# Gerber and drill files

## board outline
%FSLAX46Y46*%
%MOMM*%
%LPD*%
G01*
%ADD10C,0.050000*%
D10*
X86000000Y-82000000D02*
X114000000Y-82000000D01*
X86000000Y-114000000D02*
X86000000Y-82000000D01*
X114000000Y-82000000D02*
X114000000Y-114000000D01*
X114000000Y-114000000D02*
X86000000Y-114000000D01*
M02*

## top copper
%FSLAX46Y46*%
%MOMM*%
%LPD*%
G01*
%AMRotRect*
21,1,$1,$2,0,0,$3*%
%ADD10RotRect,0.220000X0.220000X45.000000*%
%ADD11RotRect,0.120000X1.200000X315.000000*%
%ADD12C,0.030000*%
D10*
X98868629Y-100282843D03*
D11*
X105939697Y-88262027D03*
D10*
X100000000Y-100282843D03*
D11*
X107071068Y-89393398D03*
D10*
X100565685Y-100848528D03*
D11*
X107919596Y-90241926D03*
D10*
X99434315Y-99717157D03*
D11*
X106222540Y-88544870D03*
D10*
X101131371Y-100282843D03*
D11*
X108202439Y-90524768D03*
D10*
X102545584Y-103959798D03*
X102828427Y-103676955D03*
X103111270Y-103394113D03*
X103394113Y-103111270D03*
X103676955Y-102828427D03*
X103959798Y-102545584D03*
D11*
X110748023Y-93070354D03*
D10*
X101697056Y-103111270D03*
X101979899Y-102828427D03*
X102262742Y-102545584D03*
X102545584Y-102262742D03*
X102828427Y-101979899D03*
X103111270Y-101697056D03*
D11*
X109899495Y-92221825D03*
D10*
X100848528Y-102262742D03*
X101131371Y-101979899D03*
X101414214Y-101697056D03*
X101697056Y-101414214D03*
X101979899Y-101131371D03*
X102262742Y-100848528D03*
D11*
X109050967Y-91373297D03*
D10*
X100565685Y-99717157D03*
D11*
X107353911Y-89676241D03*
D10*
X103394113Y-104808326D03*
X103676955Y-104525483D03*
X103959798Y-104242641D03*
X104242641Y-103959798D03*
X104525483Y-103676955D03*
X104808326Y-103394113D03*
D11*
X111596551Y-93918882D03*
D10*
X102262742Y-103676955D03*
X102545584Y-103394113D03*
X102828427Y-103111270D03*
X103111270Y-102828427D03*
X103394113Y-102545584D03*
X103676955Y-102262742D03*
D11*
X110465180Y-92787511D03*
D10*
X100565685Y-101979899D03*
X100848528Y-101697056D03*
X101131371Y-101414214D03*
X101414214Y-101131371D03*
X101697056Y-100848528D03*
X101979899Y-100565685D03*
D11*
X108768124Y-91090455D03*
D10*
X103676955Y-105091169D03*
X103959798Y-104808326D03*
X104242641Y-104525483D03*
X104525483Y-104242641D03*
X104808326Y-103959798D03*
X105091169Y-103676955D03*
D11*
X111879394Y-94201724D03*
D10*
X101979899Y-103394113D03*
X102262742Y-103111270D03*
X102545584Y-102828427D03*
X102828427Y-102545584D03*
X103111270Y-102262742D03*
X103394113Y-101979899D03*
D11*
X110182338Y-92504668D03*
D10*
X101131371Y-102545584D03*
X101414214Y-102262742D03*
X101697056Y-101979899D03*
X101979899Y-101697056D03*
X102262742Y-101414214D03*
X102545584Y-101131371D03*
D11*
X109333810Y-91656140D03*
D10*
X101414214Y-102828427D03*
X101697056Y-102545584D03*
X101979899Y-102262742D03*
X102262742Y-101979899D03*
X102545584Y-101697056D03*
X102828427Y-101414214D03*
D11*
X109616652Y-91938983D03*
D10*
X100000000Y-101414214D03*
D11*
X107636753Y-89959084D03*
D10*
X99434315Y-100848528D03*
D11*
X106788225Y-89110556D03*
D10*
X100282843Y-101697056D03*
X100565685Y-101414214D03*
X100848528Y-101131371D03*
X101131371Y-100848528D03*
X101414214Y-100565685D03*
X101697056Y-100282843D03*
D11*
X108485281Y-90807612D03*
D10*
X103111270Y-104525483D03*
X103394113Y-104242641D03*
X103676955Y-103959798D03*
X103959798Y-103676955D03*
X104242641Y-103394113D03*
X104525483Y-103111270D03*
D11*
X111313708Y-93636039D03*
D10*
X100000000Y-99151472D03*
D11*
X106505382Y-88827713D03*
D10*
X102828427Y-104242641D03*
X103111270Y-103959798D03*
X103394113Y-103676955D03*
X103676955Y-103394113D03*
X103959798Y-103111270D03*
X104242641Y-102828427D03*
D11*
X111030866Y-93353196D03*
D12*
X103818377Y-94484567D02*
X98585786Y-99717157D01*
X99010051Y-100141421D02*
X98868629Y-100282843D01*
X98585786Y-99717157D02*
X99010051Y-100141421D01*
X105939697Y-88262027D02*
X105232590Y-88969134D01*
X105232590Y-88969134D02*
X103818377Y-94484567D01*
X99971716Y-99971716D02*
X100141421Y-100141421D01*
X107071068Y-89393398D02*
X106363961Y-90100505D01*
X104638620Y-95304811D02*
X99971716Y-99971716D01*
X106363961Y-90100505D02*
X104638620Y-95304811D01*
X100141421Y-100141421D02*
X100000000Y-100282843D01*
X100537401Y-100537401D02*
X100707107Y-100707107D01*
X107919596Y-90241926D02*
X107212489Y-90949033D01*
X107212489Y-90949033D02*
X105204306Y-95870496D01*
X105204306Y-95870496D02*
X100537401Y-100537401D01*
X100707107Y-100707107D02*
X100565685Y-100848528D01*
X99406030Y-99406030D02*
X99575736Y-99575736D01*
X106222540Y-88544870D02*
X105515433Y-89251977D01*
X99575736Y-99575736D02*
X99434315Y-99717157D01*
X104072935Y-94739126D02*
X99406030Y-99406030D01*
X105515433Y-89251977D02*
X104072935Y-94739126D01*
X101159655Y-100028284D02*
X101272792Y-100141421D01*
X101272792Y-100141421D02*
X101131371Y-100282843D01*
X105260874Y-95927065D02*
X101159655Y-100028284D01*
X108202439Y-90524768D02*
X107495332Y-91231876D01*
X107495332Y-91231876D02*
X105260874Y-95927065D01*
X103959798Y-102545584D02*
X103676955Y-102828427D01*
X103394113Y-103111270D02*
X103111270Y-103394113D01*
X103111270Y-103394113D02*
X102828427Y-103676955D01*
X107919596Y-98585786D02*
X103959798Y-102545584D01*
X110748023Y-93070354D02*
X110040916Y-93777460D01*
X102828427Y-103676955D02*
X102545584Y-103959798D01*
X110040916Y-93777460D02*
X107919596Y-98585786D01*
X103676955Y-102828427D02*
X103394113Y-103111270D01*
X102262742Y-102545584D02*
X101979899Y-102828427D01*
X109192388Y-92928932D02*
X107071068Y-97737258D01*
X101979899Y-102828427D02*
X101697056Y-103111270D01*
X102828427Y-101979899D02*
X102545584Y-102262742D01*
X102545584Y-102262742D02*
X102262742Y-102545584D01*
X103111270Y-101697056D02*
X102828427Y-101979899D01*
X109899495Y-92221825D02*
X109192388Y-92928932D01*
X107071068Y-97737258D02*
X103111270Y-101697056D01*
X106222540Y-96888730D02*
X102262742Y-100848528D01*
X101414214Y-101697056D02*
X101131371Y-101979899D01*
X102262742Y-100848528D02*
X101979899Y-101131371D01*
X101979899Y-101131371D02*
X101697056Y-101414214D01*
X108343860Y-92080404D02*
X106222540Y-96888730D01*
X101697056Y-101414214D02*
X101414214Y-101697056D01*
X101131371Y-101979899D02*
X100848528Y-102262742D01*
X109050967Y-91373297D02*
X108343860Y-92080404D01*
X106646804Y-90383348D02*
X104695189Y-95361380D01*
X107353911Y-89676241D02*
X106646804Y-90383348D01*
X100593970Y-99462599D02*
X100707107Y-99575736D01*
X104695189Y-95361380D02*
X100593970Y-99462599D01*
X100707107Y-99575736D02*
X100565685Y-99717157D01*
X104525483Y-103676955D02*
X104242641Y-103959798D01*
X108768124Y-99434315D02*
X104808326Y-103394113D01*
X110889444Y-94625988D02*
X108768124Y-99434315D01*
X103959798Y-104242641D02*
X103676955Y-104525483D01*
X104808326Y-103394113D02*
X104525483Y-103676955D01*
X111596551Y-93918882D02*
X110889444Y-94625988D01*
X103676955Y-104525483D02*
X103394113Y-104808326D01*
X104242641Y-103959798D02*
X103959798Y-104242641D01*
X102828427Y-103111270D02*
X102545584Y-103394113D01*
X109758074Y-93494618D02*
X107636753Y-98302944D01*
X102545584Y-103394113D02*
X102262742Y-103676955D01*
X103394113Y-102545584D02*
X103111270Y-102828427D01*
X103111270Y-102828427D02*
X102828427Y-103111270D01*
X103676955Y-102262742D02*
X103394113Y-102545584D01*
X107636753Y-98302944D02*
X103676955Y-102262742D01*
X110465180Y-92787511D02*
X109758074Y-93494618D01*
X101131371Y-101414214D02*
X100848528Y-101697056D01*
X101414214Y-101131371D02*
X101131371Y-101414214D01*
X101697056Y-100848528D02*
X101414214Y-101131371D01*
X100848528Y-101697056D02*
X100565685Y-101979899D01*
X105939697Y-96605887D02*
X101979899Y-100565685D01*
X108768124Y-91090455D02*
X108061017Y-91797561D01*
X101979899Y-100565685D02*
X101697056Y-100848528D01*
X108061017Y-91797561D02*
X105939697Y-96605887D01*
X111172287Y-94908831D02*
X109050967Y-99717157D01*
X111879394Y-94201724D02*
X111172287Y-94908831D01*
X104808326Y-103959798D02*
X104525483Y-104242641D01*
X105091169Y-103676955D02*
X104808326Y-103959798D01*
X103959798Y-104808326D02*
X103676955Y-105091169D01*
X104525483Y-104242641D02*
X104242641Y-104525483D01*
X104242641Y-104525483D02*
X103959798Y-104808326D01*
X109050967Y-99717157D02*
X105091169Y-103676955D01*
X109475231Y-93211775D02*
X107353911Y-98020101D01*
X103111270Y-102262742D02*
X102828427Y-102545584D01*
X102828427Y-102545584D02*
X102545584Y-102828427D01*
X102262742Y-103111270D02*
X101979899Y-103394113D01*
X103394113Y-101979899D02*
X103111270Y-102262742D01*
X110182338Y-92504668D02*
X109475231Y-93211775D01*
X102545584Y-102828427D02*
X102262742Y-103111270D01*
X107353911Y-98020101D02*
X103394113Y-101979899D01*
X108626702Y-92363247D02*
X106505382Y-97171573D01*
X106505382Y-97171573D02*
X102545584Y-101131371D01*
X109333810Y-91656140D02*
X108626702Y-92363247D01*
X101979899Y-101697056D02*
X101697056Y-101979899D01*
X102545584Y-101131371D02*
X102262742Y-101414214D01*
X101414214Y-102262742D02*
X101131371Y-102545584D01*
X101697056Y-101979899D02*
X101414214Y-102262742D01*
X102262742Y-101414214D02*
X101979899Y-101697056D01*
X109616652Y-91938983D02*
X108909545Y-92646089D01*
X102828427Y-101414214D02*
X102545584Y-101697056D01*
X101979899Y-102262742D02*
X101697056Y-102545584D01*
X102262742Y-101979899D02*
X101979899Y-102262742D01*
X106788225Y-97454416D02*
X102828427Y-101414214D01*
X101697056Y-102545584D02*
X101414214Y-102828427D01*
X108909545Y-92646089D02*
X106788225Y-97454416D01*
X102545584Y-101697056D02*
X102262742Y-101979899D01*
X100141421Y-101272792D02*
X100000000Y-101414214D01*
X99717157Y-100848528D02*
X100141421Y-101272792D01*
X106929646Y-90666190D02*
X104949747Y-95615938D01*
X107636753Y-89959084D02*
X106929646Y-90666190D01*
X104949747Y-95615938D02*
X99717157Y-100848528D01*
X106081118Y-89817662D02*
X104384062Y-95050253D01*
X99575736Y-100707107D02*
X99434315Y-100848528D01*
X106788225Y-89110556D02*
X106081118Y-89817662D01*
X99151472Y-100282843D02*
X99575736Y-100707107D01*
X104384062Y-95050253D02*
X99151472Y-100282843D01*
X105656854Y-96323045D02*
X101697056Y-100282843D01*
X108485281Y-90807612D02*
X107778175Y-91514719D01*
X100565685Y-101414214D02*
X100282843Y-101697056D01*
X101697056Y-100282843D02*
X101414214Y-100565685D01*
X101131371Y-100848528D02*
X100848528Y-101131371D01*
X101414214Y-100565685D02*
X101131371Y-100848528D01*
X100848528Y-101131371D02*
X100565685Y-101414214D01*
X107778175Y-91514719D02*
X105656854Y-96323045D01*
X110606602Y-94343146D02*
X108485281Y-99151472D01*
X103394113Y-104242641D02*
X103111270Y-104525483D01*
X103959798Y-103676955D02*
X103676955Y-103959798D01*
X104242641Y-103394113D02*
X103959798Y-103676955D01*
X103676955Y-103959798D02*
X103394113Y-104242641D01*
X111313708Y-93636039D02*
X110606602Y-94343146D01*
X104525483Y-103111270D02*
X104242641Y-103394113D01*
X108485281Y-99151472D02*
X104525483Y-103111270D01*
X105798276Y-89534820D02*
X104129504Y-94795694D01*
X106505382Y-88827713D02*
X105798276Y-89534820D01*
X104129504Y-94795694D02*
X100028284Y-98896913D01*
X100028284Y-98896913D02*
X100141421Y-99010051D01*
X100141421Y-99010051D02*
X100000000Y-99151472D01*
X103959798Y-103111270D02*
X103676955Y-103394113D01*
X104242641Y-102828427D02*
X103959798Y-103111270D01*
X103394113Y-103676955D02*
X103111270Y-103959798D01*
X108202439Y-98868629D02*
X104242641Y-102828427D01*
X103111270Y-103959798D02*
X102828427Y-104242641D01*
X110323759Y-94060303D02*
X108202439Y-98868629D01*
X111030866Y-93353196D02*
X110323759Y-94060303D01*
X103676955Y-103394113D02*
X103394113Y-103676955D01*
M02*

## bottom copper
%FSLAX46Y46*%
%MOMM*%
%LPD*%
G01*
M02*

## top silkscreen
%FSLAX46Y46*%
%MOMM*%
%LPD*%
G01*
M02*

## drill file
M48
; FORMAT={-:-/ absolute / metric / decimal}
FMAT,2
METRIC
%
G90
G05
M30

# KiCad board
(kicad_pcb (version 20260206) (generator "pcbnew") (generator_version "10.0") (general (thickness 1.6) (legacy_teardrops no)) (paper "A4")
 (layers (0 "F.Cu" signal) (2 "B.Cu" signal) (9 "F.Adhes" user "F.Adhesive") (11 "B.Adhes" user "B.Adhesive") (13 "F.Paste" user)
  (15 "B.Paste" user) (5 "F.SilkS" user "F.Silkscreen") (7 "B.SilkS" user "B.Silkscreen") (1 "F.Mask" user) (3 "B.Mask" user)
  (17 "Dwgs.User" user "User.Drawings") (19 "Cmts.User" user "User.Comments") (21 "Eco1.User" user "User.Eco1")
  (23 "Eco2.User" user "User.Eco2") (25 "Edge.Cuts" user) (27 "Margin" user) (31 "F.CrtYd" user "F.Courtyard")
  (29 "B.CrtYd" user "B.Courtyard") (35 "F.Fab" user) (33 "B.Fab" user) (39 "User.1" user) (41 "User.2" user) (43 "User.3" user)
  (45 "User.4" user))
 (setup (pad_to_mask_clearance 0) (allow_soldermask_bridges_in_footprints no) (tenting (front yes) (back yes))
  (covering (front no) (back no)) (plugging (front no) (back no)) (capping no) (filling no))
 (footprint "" (layer "F.Cu") (at 0 0)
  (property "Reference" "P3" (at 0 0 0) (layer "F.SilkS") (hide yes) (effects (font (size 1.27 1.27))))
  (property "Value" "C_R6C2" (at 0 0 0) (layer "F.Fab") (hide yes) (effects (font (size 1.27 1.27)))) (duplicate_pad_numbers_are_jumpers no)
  (pad "1" connect rect (at 98.868629 100.282843 45) (size 0.22 0.22) (layers "F.Cu") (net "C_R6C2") (thermal_bridge_angle 45))
  (pad "2" connect rect (at 105.939697 88.262027 315) (size 0.12 1.2) (layers "F.Cu") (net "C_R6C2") (thermal_bridge_angle 45)))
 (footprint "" (layer "F.Cu") (at 0 0)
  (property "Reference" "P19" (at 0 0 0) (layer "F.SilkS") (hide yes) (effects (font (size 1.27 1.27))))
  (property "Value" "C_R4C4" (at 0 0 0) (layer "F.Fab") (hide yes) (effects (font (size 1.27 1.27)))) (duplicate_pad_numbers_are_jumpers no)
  (pad "1" connect rect (at 100 100.282843 45) (size 0.22 0.22) (layers "F.Cu") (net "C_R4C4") (thermal_bridge_angle 45))
  (pad "2" connect rect (at 107.071068 89.393398 315) (size 0.12 1.2) (layers "F.Cu") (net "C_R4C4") (thermal_bridge_angle 45)))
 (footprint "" (layer "F.Cu") (at 0 0)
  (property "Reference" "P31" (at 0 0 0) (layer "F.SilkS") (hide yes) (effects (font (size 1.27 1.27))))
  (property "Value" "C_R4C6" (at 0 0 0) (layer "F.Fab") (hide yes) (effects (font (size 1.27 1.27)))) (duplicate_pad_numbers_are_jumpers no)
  (pad "1" connect rect (at 100.565685 100.848528 45) (size 0.22 0.22) (layers "F.Cu") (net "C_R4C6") (thermal_bridge_angle 45))
  (pad "2" connect rect (at 107.919596 90.241926 315) (size 0.12 1.2) (layers "F.Cu") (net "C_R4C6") (thermal_bridge_angle 45)))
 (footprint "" (layer "F.Cu") (at 0 0)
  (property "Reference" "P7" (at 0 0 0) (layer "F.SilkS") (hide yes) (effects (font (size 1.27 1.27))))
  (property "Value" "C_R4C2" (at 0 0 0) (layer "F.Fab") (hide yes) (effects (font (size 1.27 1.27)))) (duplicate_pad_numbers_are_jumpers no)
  (pad "1" connect rect (at 99.434315 99.717157 45) (size 0.22 0.22) (layers "F.Cu") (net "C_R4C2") (thermal_bridge_angle 45))
  (pad "2" connect rect (at 106.22254 88.54487 315) (size 0.12 1.2) (layers "F.Cu") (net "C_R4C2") (thermal_bridge_angle 45)))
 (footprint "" (layer "F.Cu") (at 0 0)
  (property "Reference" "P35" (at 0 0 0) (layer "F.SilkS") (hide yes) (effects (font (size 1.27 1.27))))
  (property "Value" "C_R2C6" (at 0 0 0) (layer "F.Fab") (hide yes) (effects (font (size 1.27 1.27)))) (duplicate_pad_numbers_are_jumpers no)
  (pad "1" connect rect (at 101.131371 100.282843 45) (size 0.22 0.22) (layers "F.Cu") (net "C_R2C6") (thermal_bridge_angle 45))
  (pad "2" connect rect (at 108.202439 90.524768 315) (size 0.12 1.2) (layers "F.Cu") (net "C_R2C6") (thermal_bridge_angle 45)))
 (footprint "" (layer "F.Cu") (at 0 0)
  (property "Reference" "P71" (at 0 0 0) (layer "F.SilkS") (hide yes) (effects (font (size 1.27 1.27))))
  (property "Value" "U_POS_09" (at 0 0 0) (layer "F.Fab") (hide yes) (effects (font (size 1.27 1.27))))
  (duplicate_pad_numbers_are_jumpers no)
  (pad "1" connect rect (at 102.545584 103.959798 45) (size 0.22 0.22) (layers "F.Cu") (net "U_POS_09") (thermal_bridge_angle 45))
  (pad "1" connect rect (at 102.828427 103.676955 45) (size 0.22 0.22) (layers "F.Cu") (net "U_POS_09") (thermal_bridge_angle 45))
  (pad "1" connect rect (at 103.11127 103.394113 45) (size 0.22 0.22) (layers "F.Cu") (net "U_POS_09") (thermal_bridge_angle 45))
  (pad "1" connect rect (at 103.394113 103.11127 45) (size 0.22 0.22) (layers "F.Cu") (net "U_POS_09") (thermal_bridge_angle 45))
  (pad "1" connect rect (at 103.676955 102.828427 45) (size 0.22 0.22) (layers "F.Cu") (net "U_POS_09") (thermal_bridge_angle 45))
  (pad "1" connect rect (at 103.959798 102.545584 45) (size 0.22 0.22) (layers "F.Cu") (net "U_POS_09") (thermal_bridge_angle 45))
  (pad "2" connect rect (at 110.748023 93.070354 315) (size 0.12 1.2) (layers "F.Cu") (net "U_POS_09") (thermal_bridge_angle 45)))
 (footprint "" (layer "F.Cu") (at 0 0)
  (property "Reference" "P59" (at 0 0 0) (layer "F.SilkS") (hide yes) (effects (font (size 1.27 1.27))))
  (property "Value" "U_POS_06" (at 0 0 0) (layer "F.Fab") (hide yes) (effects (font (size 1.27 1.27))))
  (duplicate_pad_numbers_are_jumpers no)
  (pad "1" connect rect (at 101.697056 103.11127 45) (size 0.22 0.22) (layers "F.Cu") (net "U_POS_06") (thermal_bridge_angle 45))
  (pad "1" connect rect (at 101.979899 102.828427 45) (size 0.22 0.22) (layers "F.Cu") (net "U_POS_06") (thermal_bridge_angle 45))
  (pad "1" connect rect (at 102.262742 102.545584 45) (size 0.22 0.22) (layers "F.Cu") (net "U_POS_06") (thermal_bridge_angle 45))
  (pad "1" connect rect (at 102.545584 102.262742 45) (size 0.22 0.22) (layers "F.Cu") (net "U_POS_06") (thermal_bridge_angle 45))
  (pad "1" connect rect (at 102.828427 101.979899 45) (size 0.22 0.22) (layers "F.Cu") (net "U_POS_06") (thermal_bridge_angle 45))
  (pad "1" connect rect (at 103.11127 101.697056 45) (size 0.22 0.22) (layers "F.Cu") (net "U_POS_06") (thermal_bridge_angle 45))
  (pad "2" connect rect (at 109.899495 92.221825 315) (size 0.12 1.2) (layers "F.Cu") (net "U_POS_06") (thermal_bridge_angle 45)))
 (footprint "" (layer "F.Cu") (at 0 0)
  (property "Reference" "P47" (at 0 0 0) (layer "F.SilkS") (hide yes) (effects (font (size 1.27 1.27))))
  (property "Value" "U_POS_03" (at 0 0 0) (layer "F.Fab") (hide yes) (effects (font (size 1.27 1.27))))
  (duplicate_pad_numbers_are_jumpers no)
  (pad "1" connect rect (at 100.848528 102.262742 45) (size 0.22 0.22) (layers "F.Cu") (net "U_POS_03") (thermal_bridge_angle 45))
  (pad "1" connect rect (at 101.131371 101.979899 45) (size 0.22 0.22) (layers "F.Cu") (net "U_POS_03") (thermal_bridge_angle 45))
  (pad "1" connect rect (at 101.414214 101.697056 45) (size 0.22 0.22) (layers "F.Cu") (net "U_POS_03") (thermal_bridge_angle 45))
  (pad "1" connect rect (at 101.697056 101.414214 45) (size 0.22 0.22) (layers "F.Cu") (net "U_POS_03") (thermal_bridge_angle 45))
  (pad "1" connect rect (at 101.979899 101.131371 45) (size 0.22 0.22) (layers "F.Cu") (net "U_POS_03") (thermal_bridge_angle 45))
  (pad "1" connect rect (at 102.262742 100.848528 45) (size 0.22 0.22) (layers "F.Cu") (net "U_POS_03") (thermal_bridge_angle 45))
  (pad "2" connect rect (at 109.050967 91.373297 315) (size 0.12 1.2) (layers "F.Cu") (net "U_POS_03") (thermal_bridge_angle 45)))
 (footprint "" (layer "F.Cu") (at 0 0)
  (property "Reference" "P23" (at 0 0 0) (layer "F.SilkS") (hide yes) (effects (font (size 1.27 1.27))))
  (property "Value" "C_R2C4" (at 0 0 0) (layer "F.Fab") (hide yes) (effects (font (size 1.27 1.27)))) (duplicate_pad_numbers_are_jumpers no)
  (pad "1" connect rect (at 100.565685 99.717157 45) (size 0.22 0.22) (layers "F.Cu") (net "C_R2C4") (thermal_bridge_angle 45))
  (pad "2" connect rect (at 107.353911 89.676241 315) (size 0.12 1.2) (layers "F.Cu") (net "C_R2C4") (thermal_bridge_angle 45)))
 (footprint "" (layer "F.Cu") (at 0 0)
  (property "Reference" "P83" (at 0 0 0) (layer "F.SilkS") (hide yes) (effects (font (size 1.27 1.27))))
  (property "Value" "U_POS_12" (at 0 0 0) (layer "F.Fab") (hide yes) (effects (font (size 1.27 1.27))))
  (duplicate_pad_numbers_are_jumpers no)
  (pad "1" connect rect (at 103.394113 104.808326 45) (size 0.22 0.22) (layers "F.Cu") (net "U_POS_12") (thermal_bridge_angle 45))
  (pad "1" connect rect (at 103.676955 104.525483 45) (size 0.22 0.22) (layers "F.Cu") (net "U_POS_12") (thermal_bridge_angle 45))
  (pad "1" connect rect (at 103.959798 104.242641 45) (size 0.22 0.22) (layers "F.Cu") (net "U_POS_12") (thermal_bridge_angle 45))
  (pad "1" connect rect (at 104.242641 103.959798 45) (size 0.22 0.22) (layers "F.Cu") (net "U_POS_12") (thermal_bridge_angle 45))
  (pad "1" connect rect (at 104.525483 103.676955 45) (size 0.22 0.22) (layers "F.Cu") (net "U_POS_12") (thermal_bridge_angle 45))
  (pad "1" connect rect (at 104.808326 103.394113 45) (size 0.22 0.22) (layers "F.Cu") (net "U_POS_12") (thermal_bridge_angle 45))
  (pad "2" connect rect (at 111.596551 93.918882 315) (size 0.12 1.2) (layers "F.Cu") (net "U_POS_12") (thermal_bridge_angle 45)))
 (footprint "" (layer "F.Cu") (at 0 0)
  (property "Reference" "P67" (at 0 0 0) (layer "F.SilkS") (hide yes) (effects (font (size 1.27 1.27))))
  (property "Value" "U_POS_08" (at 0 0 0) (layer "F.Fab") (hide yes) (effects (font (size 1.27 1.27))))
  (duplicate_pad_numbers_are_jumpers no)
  (pad "1" connect rect (at 102.262742 103.676955 45) (size 0.22 0.22) (layers "F.Cu") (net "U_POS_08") (thermal_bridge_angle 45))
  (pad "1" connect rect (at 102.545584 103.394113 45) (size 0.22 0.22) (layers "F.Cu") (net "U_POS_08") (thermal_bridge_angle 45))
  (pad "1" connect rect (at 102.828427 103.11127 45) (size 0.22 0.22) (layers "F.Cu") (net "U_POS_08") (thermal_bridge_angle 45))
  (pad "1" connect rect (at 103.11127 102.828427 45) (size 0.22 0.22) (layers "F.Cu") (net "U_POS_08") (thermal_bridge_angle 45))
  (pad "1" connect rect (at 103.394113 102.545584 45) (size 0.22 0.22) (layers "F.Cu") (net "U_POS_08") (thermal_bridge_angle 45))
  (pad "1" connect rect (at 103.676955 102.262742 45) (size 0.22 0.22) (layers "F.Cu") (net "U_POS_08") (thermal_bridge_angle 45))
  (pad "2" connect rect (at 110.46518 92.787511 315) (size 0.12 1.2) (layers "F.Cu") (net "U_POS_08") (thermal_bridge_angle 45)))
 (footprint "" (layer "F.Cu") (at 0 0)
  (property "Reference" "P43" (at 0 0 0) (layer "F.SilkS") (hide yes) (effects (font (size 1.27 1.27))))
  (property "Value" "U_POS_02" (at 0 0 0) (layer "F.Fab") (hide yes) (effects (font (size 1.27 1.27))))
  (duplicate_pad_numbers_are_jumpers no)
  (pad "1" connect rect (at 100.565685 101.979899 45) (size 0.22 0.22) (layers "F.Cu") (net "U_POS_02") (thermal_bridge_angle 45))
  (pad "1" connect rect (at 100.848528 101.697056 45) (size 0.22 0.22) (layers "F.Cu") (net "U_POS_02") (thermal_bridge_angle 45))
  (pad "1" connect rect (at 101.131371 101.414214 45) (size 0.22 0.22) (layers "F.Cu") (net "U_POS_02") (thermal_bridge_angle 45))
  (pad "1" connect rect (at 101.414214 101.131371 45) (size 0.22 0.22) (layers "F.Cu") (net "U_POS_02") (thermal_bridge_angle 45))
  (pad "1" connect rect (at 101.697056 100.848528 45) (size 0.22 0.22) (layers "F.Cu") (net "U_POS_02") (thermal_bridge_angle 45))
  (pad "1" connect rect (at 101.979899 100.565685 45) (size 0.22 0.22) (layers "F.Cu") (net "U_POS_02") (thermal_bridge_angle 45))
  (pad "2" connect rect (at 108.768124 91.090455 315) (size 0.12 1.2) (layers "F.Cu") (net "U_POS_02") (thermal_bridge_angle 45)))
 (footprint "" (layer "F.Cu") (at 0 0)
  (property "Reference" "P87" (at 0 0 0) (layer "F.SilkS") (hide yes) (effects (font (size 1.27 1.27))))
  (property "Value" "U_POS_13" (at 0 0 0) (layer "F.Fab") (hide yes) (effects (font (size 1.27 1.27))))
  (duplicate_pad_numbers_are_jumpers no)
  (pad "1" connect rect (at 103.676955 105.091169 45) (size 0.22 0.22) (layers "F.Cu") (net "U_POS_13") (thermal_bridge_angle 45))
  (pad "1" connect rect (at 103.959798 104.808326 45) (size 0.22 0.22) (layers "F.Cu") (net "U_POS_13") (thermal_bridge_angle 45))
  (pad "1" connect rect (at 104.242641 104.525483 45) (size 0.22 0.22) (layers "F.Cu") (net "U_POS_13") (thermal_bridge_angle 45))
  (pad "1" connect rect (at 104.525483 104.242641 45) (size 0.22 0.22) (layers "F.Cu") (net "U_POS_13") (thermal_bridge_angle 45))
  (pad "1" connect rect (at 104.808326 103.959798 45) (size 0.22 0.22) (layers "F.Cu") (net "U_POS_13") (thermal_bridge_angle 45))
  (pad "1" connect rect (at 105.091169 103.676955 45) (size 0.22 0.22) (layers "F.Cu") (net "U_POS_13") (thermal_bridge_angle 45))
  (pad "2" connect rect (at 111.879394 94.201724 315) (size 0.12 1.2) (layers "F.Cu") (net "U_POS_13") (thermal_bridge_angle 45)))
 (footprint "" (layer "F.Cu") (at 0 0)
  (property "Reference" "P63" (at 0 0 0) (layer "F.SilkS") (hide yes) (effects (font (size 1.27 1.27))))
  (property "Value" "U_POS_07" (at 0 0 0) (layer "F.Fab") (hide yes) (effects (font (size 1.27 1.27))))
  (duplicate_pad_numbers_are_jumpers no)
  (pad "1" connect rect (at 101.979899 103.394113 45) (size 0.22 0.22) (layers "F.Cu") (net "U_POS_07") (thermal_bridge_angle 45))
  (pad "1" connect rect (at 102.262742 103.11127 45) (size 0.22 0.22) (layers "F.Cu") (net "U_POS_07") (thermal_bridge_angle 45))
  (pad "1" connect rect (at 102.545584 102.828427 45) (size 0.22 0.22) (layers "F.Cu") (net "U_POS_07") (thermal_bridge_angle 45))
  (pad "1" connect rect (at 102.828427 102.545584 45) (size 0.22 0.22) (layers "F.Cu") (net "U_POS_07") (thermal_bridge_angle 45))
  (pad "1" connect rect (at 103.11127 102.262742 45) (size 0.22 0.22) (layers "F.Cu") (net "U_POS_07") (thermal_bridge_angle 45))
  (pad "1" connect rect (at 103.394113 101.979899 45) (size 0.22 0.22) (layers "F.Cu") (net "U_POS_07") (thermal_bridge_angle 45))
  (pad "2" connect rect (at 110.182338 92.504668 315) (size 0.12 1.2) (layers "F.Cu") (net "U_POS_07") (thermal_bridge_angle 45)))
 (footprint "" (layer "F.Cu") (at 0 0)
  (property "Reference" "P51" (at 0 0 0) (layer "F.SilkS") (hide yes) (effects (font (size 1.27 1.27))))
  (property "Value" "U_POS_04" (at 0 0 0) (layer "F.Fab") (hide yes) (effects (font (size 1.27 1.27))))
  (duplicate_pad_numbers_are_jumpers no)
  (pad "1" connect rect (at 101.131371 102.545584 45) (size 0.22 0.22) (layers "F.Cu") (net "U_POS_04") (thermal_bridge_angle 45))
  (pad "1" connect rect (at 101.414214 102.262742 45) (size 0.22 0.22) (layers "F.Cu") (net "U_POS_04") (thermal_bridge_angle 45))
  (pad "1" connect rect (at 101.697056 101.979899 45) (size 0.22 0.22) (layers "F.Cu") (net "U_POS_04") (thermal_bridge_angle 45))
  (pad "1" connect rect (at 101.979899 101.697056 45) (size 0.22 0.22) (layers "F.Cu") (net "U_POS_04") (thermal_bridge_angle 45))
  (pad "1" connect rect (at 102.262742 101.414214 45) (size 0.22 0.22) (layers "F.Cu") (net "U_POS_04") (thermal_bridge_angle 45))
  (pad "1" connect rect (at 102.545584 101.131371 45) (size 0.22 0.22) (layers "F.Cu") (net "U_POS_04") (thermal_bridge_angle 45))
  (pad "2" connect rect (at 109.33381 91.65614 315) (size 0.12 1.2) (layers "F.Cu") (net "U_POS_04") (thermal_bridge_angle 45)))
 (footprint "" (layer "F.Cu") (at 0 0)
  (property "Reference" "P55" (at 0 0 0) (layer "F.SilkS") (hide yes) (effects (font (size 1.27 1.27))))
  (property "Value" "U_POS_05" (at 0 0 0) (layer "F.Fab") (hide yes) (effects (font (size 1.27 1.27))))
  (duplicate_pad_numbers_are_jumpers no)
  (pad "1" connect rect (at 101.414214 102.828427 45) (size 0.22 0.22) (layers "F.Cu") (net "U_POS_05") (thermal_bridge_angle 45))
  (pad "1" connect rect (at 101.697056 102.545584 45) (size 0.22 0.22) (layers "F.Cu") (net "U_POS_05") (thermal_bridge_angle 45))
  (pad "1" connect rect (at 101.979899 102.262742 45) (size 0.22 0.22) (layers "F.Cu") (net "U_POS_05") (thermal_bridge_angle 45))
  (pad "1" connect rect (at 102.262742 101.979899 45) (size 0.22 0.22) (layers "F.Cu") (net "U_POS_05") (thermal_bridge_angle 45))
  (pad "1" connect rect (at 102.545584 101.697056 45) (size 0.22 0.22) (layers "F.Cu") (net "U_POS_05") (thermal_bridge_angle 45))
  (pad "1" connect rect (at 102.828427 101.414214 45) (size 0.22 0.22) (layers "F.Cu") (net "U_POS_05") (thermal_bridge_angle 45))
  (pad "2" connect rect (at 109.616652 91.938983 315) (size 0.12 1.2) (layers "F.Cu") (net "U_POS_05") (thermal_bridge_angle 45)))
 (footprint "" (layer "F.Cu") (at 0 0)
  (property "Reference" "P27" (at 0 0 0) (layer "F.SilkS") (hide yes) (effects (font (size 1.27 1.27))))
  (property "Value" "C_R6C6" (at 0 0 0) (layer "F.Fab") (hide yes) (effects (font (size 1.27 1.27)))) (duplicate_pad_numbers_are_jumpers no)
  (pad "1" connect rect (at 100 101.414214 45) (size 0.22 0.22) (layers "F.Cu") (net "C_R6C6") (thermal_bridge_angle 45))
  (pad "2" connect rect (at 107.636753 89.959084 315) (size 0.12 1.2) (layers "F.Cu") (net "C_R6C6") (thermal_bridge_angle 45)))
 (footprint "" (layer "F.Cu") (at 0 0)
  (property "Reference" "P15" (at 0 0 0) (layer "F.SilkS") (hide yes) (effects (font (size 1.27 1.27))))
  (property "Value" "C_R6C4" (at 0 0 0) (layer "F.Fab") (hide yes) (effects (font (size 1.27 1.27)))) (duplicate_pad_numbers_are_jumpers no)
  (pad "1" connect rect (at 99.434315 100.848528 45) (size 0.22 0.22) (layers "F.Cu") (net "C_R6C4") (thermal_bridge_angle 45))
  (pad "2" connect rect (at 106.788225 89.110556 315) (size 0.12 1.2) (layers "F.Cu") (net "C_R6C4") (thermal_bridge_angle 45)))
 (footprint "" (layer "F.Cu") (at 0 0)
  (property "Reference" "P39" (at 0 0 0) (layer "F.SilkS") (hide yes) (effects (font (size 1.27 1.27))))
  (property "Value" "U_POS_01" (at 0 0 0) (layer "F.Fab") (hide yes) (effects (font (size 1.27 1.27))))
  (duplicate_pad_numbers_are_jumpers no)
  (pad "1" connect rect (at 100.282843 101.697056 45) (size 0.22 0.22) (layers "F.Cu") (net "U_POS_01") (thermal_bridge_angle 45))
  (pad "1" connect rect (at 100.565685 101.414214 45) (size 0.22 0.22) (layers "F.Cu") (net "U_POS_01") (thermal_bridge_angle 45))
  (pad "1" connect rect (at 100.848528 101.131371 45) (size 0.22 0.22) (layers "F.Cu") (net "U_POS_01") (thermal_bridge_angle 45))
  (pad "1" connect rect (at 101.131371 100.848528 45) (size 0.22 0.22) (layers "F.Cu") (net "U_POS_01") (thermal_bridge_angle 45))
  (pad "1" connect rect (at 101.414214 100.565685 45) (size 0.22 0.22) (layers "F.Cu") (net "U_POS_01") (thermal_bridge_angle 45))
  (pad "1" connect rect (at 101.697056 100.282843 45) (size 0.22 0.22) (layers "F.Cu") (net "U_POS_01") (thermal_bridge_angle 45))
  (pad "2" connect rect (at 108.485281 90.807612 315) (size 0.12 1.2) (layers "F.Cu") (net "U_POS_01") (thermal_bridge_angle 45)))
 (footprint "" (layer "F.Cu") (at 0 0)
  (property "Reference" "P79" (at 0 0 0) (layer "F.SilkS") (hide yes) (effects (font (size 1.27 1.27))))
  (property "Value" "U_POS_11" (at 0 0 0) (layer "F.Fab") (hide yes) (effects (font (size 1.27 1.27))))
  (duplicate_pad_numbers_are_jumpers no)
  (pad "1" connect rect (at 103.11127 104.525483 45) (size 0.22 0.22) (layers "F.Cu") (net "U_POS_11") (thermal_bridge_angle 45))
  (pad "1" connect rect (at 103.394113 104.242641 45) (size 0.22 0.22) (layers "F.Cu") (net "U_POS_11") (thermal_bridge_angle 45))
  (pad "1" connect rect (at 103.676955 103.959798 45) (size 0.22 0.22) (layers "F.Cu") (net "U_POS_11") (thermal_bridge_angle 45))
  (pad "1" connect rect (at 103.959798 103.676955 45) (size 0.22 0.22) (layers "F.Cu") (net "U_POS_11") (thermal_bridge_angle 45))
  (pad "1" connect rect (at 104.242641 103.394113 45) (size 0.22 0.22) (layers "F.Cu") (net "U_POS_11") (thermal_bridge_angle 45))
  (pad "1" connect rect (at 104.525483 103.11127 45) (size 0.22 0.22) (layers "F.Cu") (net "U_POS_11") (thermal_bridge_angle 45))
  (pad "2" connect rect (at 111.313708 93.636039 315) (size 0.12 1.2) (layers "F.Cu") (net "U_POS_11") (thermal_bridge_angle 45)))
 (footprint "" (layer "F.Cu") (at 0 0)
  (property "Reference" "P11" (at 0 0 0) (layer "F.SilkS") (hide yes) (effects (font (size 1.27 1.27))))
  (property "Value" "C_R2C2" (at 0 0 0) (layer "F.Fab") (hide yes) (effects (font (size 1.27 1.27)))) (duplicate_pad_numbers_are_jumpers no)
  (pad "1" connect rect (at 100 99.151472 45) (size 0.22 0.22) (layers "F.Cu") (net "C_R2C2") (thermal_bridge_angle 45))
  (pad "2" connect rect (at 106.505382 88.827713 315) (size 0.12 1.2) (layers "F.Cu") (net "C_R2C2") (thermal_bridge_angle 45)))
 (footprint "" (layer "F.Cu") (at 0 0)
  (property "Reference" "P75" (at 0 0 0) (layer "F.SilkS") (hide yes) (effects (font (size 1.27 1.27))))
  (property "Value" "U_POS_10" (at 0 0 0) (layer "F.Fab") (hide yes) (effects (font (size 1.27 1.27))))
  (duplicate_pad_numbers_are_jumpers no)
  (pad "1" connect rect (at 102.828427 104.242641 45) (size 0.22 0.22) (layers "F.Cu") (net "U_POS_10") (thermal_bridge_angle 45))
  (pad "1" connect rect (at 103.11127 103.959798 45) (size 0.22 0.22) (layers "F.Cu") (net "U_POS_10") (thermal_bridge_angle 45))
  (pad "1" connect rect (at 103.394113 103.676955 45) (size 0.22 0.22) (layers "F.Cu") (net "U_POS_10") (thermal_bridge_angle 45))
  (pad "1" connect rect (at 103.676955 103.394113 45) (size 0.22 0.22) (layers "F.Cu") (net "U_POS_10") (thermal_bridge_angle 45))
  (pad "1" connect rect (at 103.959798 103.11127 45) (size 0.22 0.22) (layers "F.Cu") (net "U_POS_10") (thermal_bridge_angle 45))
  (pad "1" connect rect (at 104.242641 102.828427 45) (size 0.22 0.22) (layers "F.Cu") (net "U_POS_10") (thermal_bridge_angle 45))
  (pad "2" connect rect (at 111.030866 93.353196 315) (size 0.12 1.2) (layers "F.Cu") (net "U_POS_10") (thermal_bridge_angle 45)))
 (gr_line (start 86 82) (end 114 82) (stroke (width 0.05) (type default)) (layer "Edge.Cuts"))
 (gr_line (start 86 114) (end 86 82) (stroke (width 0.05) (type default)) (layer "Edge.Cuts"))
 (gr_line (start 114 82) (end 114 114) (stroke (width 0.05) (type default)) (layer "Edge.Cuts"))
 (gr_line (start 114 114) (end 86 114) (stroke (width 0.05) (type default)) (layer "Edge.Cuts"))
 (segment (start 103.818377 94.484567) (end 98.585786 99.717157) (width 0.03) (layer "F.Cu") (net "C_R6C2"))
 (segment (start 99.010051 100.141421) (end 98.868629 100.282843) (width 0.03) (layer "F.Cu") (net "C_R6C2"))
 (segment (start 98.585786 99.717157) (end 99.010051 100.141421) (width 0.03) (layer "F.Cu") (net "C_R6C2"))
 (segment (start 105.939697 88.262027) (end 105.23259 88.969134) (width 0.03) (layer "F.Cu") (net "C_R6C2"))
 (segment (start 105.23259 88.969134) (end 103.818377 94.484567) (width 0.03) (layer "F.Cu") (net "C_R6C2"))
 (segment (start 99.971716 99.971716) (end 100.141421 100.141421) (width 0.03) (layer "F.Cu") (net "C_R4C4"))
 (segment (start 107.071068 89.393398) (end 106.363961 90.100505) (width 0.03) (layer "F.Cu") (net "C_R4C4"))
 (segment (start 104.63862 95.304811) (end 99.971716 99.971716) (width 0.03) (layer "F.Cu") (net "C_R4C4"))
 (segment (start 106.363961 90.100505) (end 104.63862 95.304811) (width 0.03) (layer "F.Cu") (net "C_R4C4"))
 (segment (start 100.141421 100.141421) (end 100 100.282843) (width 0.03) (layer "F.Cu") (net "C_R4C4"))
 (segment (start 100.537401 100.537401) (end 100.707107 100.707107) (width 0.03) (layer "F.Cu") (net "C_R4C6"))
 (segment (start 107.919596 90.241926) (end 107.212489 90.949033) (width 0.03) (layer "F.Cu") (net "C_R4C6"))
 (segment (start 107.212489 90.949033) (end 105.204306 95.870496) (width 0.03) (layer "F.Cu") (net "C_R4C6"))
 (segment (start 105.204306 95.870496) (end 100.537401 100.537401) (width 0.03) (layer "F.Cu") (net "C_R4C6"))
 (segment (start 100.707107 100.707107) (end 100.565685 100.848528) (width 0.03) (layer "F.Cu") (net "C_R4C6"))
 (segment (start 99.40603 99.40603) (end 99.575736 99.575736) (width 0.03) (layer "F.Cu") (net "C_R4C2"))
 (segment (start 106.22254 88.54487) (end 105.515433 89.251977) (width 0.03) (layer "F.Cu") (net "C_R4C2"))
 (segment (start 99.575736 99.575736) (end 99.434315 99.717157) (width 0.03) (layer "F.Cu") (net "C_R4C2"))
 (segment (start 104.072935 94.739126) (end 99.40603 99.40603) (width 0.03) (layer "F.Cu") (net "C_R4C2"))
 (segment (start 105.515433 89.251977) (end 104.072935 94.739126) (width 0.03) (layer "F.Cu") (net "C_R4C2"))
 (segment (start 101.159655 100.028284) (end 101.272792 100.141421) (width 0.03) (layer "F.Cu") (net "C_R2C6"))
 (segment (start 101.272792 100.141421) (end 101.131371 100.282843) (width 0.03) (layer "F.Cu") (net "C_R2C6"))
 (segment (start 105.260874 95.927065) (end 101.159655 100.028284) (width 0.03) (layer "F.Cu") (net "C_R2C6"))
 (segment (start 108.202439 90.524768) (end 107.495332 91.231876) (width 0.03) (layer "F.Cu") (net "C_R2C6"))
 (segment (start 107.495332 91.231876) (end 105.260874 95.927065) (width 0.03) (layer "F.Cu") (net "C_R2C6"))
 (segment (start 103.959798 102.545584) (end 103.676955 102.828427) (width 0.03) (layer "F.Cu") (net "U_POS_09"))
 (segment (start 103.394113 103.11127) (end 103.11127 103.394113) (width 0.03) (layer "F.Cu") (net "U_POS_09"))
 (segment (start 103.11127 103.394113) (end 102.828427 103.676955) (width 0.03) (layer "F.Cu") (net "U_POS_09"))
 (segment (start 107.919596 98.585786) (end 103.959798 102.545584) (width 0.03) (layer "F.Cu") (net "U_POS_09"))
 (segment (start 110.748023 93.070354) (end 110.040916 93.77746) (width 0.03) (layer "F.Cu") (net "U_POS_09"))
 (segment (start 102.828427 103.676955) (end 102.545584 103.959798) (width 0.03) (layer "F.Cu") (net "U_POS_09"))
 (segment (start 110.040916 93.77746) (end 107.919596 98.585786) (width 0.03) (layer "F.Cu") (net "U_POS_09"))
 (segment (start 103.676955 102.828427) (end 103.394113 103.11127) (width 0.03) (layer "F.Cu") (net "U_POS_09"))
 (segment (start 102.262742 102.545584) (end 101.979899 102.828427) (width 0.03) (layer "F.Cu") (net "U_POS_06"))
 (segment (start 109.192388 92.928932) (end 107.071068 97.737258) (width 0.03) (layer "F.Cu") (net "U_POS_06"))
 (segment (start 101.979899 102.828427) (end 101.697056 103.11127) (width 0.03) (layer "F.Cu") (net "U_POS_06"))
 (segment (start 102.828427 101.979899) (end 102.545584 102.262742) (width 0.03) (layer "F.Cu") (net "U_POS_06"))
 (segment (start 102.545584 102.262742) (end 102.262742 102.545584) (width 0.03) (layer "F.Cu") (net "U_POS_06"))
 (segment (start 103.11127 101.697056) (end 102.828427 101.979899) (width 0.03) (layer "F.Cu") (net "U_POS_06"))
 (segment (start 109.899495 92.221825) (end 109.192388 92.928932) (width 0.03) (layer "F.Cu") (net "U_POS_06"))
 (segment (start 107.071068 97.737258) (end 103.11127 101.697056) (width 0.03) (layer "F.Cu") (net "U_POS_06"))
 (segment (start 106.22254 96.88873) (end 102.262742 100.848528) (width 0.03) (layer "F.Cu") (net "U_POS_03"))
 (segment (start 101.414214 101.697056) (end 101.131371 101.979899) (width 0.03) (layer "F.Cu") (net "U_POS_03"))
 (segment (start 102.262742 100.848528) (end 101.979899 101.131371) (width 0.03) (layer "F.Cu") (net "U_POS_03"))
 (segment (start 101.979899 101.131371) (end 101.697056 101.414214) (width 0.03) (layer "F.Cu") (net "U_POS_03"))
 (segment (start 108.34386 92.080404) (end 106.22254 96.88873) (width 0.03) (layer "F.Cu") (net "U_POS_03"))
 (segment (start 101.697056 101.414214) (end 101.414214 101.697056) (width 0.03) (layer "F.Cu") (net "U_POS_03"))
 (segment (start 101.131371 101.979899) (end 100.848528 102.262742) (width 0.03) (layer "F.Cu") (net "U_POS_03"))
 (segment (start 109.050967 91.373297) (end 108.34386 92.080404) (width 0.03) (layer "F.Cu") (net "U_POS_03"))
 (segment (start 106.646804 90.383348) (end 104.695189 95.36138) (width 0.03) (layer "F.Cu") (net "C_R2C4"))
 (segment (start 107.353911 89.676241) (end 106.646804 90.383348) (width 0.03) (layer "F.Cu") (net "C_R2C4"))
 (segment (start 100.59397 99.462599) (end 100.707107 99.575736) (width 0.03) (layer "F.Cu") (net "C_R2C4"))
 (segment (start 104.695189 95.36138) (end 100.59397 99.462599) (width 0.03) (layer "F.Cu") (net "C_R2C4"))
 (segment (start 100.707107 99.575736) (end 100.565685 99.717157) (width 0.03) (layer "F.Cu") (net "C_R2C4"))
 (segment (start 104.525483 103.676955) (end 104.242641 103.959798) (width 0.03) (layer "F.Cu") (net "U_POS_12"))
 (segment (start 108.768124 99.434315) (end 104.808326 103.394113) (width 0.03) (layer "F.Cu") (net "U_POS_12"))
 (segment (start 110.889444 94.625988) (end 108.768124 99.434315) (width 0.03) (layer "F.Cu") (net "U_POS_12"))
 (segment (start 103.959798 104.242641) (end 103.676955 104.525483) (width 0.03) (layer "F.Cu") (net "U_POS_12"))
 (segment (start 104.808326 103.394113) (end 104.525483 103.676955) (width 0.03) (layer "F.Cu") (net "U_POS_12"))
 (segment (start 111.596551 93.918882) (end 110.889444 94.625988) (width 0.03) (layer "F.Cu") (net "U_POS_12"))
 (segment (start 103.676955 104.525483) (end 103.394113 104.808326) (width 0.03) (layer "F.Cu") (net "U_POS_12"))
 (segment (start 104.242641 103.959798) (end 103.959798 104.242641) (width 0.03) (layer "F.Cu") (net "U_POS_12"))
 (segment (start 102.828427 103.11127) (end 102.545584 103.394113) (width 0.03) (layer "F.Cu") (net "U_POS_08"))
 (segment (start 109.758074 93.494618) (end 107.636753 98.302944) (width 0.03) (layer "F.Cu") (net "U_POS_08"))
 (segment (start 102.545584 103.394113) (end 102.262742 103.676955) (width 0.03) (layer "F.Cu") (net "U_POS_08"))
 (segment (start 103.394113 102.545584) (end 103.11127 102.828427) (width 0.03) (layer "F.Cu") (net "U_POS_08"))
 (segment (start 103.11127 102.828427) (end 102.828427 103.11127) (width 0.03) (layer "F.Cu") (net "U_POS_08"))
 (segment (start 103.676955 102.262742) (end 103.394113 102.545584) (width 0.03) (layer "F.Cu") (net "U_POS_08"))
 (segment (start 107.636753 98.302944) (end 103.676955 102.262742) (width 0.03) (layer "F.Cu") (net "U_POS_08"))
 (segment (start 110.46518 92.787511) (end 109.758074 93.494618) (width 0.03) (layer "F.Cu") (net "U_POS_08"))
 (segment (start 101.131371 101.414214) (end 100.848528 101.697056) (width 0.03) (layer "F.Cu") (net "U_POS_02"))
 (segment (start 101.414214 101.131371) (end 101.131371 101.414214) (width 0.03) (layer "F.Cu") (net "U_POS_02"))
 (segment (start 101.697056 100.848528) (end 101.414214 101.131371) (width 0.03) (layer "F.Cu") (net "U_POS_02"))
 (segment (start 100.848528 101.697056) (end 100.565685 101.979899) (width 0.03) (layer "F.Cu") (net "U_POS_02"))
 (segment (start 105.939697 96.605887) (end 101.979899 100.565685) (width 0.03) (layer "F.Cu") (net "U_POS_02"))
 (segment (start 108.768124 91.090455) (end 108.061017 91.797561) (width 0.03) (layer "F.Cu") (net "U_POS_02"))
 (segment (start 101.979899 100.565685) (end 101.697056 100.848528) (width 0.03) (layer "F.Cu") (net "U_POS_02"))
 (segment (start 108.061017 91.797561) (end 105.939697 96.605887) (width 0.03) (layer "F.Cu") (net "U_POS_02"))
 (segment (start 111.172287 94.908831) (end 109.050967 99.717157) (width 0.03) (layer "F.Cu") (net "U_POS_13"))
 (segment (start 111.879394 94.201724) (end 111.172287 94.908831) (width 0.03) (layer "F.Cu") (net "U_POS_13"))
 (segment (start 104.808326 103.959798) (end 104.525483 104.242641) (width 0.03) (layer "F.Cu") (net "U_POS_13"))
 (segment (start 105.091169 103.676955) (end 104.808326 103.959798) (width 0.03) (layer "F.Cu") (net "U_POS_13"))
 (segment (start 103.959798 104.808326) (end 103.676955 105.091169) (width 0.03) (layer "F.Cu") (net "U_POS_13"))
 (segment (start 104.525483 104.242641) (end 104.242641 104.525483) (width 0.03) (layer "F.Cu") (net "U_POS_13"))
 (segment (start 104.242641 104.525483) (end 103.959798 104.808326) (width 0.03) (layer "F.Cu") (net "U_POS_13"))
 (segment (start 109.050967 99.717157) (end 105.091169 103.676955) (width 0.03) (layer "F.Cu") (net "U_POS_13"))
 (segment (start 109.475231 93.211775) (end 107.353911 98.020101) (width 0.03) (layer "F.Cu") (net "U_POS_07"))
 (segment (start 103.11127 102.262742) (end 102.828427 102.545584) (width 0.03) (layer "F.Cu") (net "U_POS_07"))
 (segment (start 102.828427 102.545584) (end 102.545584 102.828427) (width 0.03) (layer "F.Cu") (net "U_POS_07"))
 (segment (start 102.262742 103.11127) (end 101.979899 103.394113) (width 0.03) (layer "F.Cu") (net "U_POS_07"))
 (segment (start 103.394113 101.979899) (end 103.11127 102.262742) (width 0.03) (layer "F.Cu") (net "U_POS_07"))
 (segment (start 110.182338 92.504668) (end 109.475231 93.211775) (width 0.03) (layer "F.Cu") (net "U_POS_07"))
 (segment (start 102.545584 102.828427) (end 102.262742 103.11127) (width 0.03) (layer "F.Cu") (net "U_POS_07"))
 (segment (start 107.353911 98.020101) (end 103.394113 101.979899) (width 0.03) (layer "F.Cu") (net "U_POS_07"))
 (segment (start 108.626702 92.363247) (end 106.505382 97.171573) (width 0.03) (layer "F.Cu") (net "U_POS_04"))
 (segment (start 106.505382 97.171573) (end 102.545584 101.131371) (width 0.03) (layer "F.Cu") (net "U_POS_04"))
 (segment (start 109.33381 91.65614) (end 108.626702 92.363247) (width 0.03) (layer "F.Cu") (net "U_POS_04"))
 (segment (start 101.979899 101.697056) (end 101.697056 101.979899) (width 0.03) (layer "F.Cu") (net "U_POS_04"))
 (segment (start 102.545584 101.131371) (end 102.262742 101.414214) (width 0.03) (layer "F.Cu") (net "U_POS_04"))
 (segment (start 101.414214 102.262742) (end 101.131371 102.545584) (width 0.03) (layer "F.Cu") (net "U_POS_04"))
 (segment (start 101.697056 101.979899) (end 101.414214 102.262742) (width 0.03) (layer "F.Cu") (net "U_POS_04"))
 (segment (start 102.262742 101.414214) (end 101.979899 101.697056) (width 0.03) (layer "F.Cu") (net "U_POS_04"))
 (segment (start 109.616652 91.938983) (end 108.909545 92.646089) (width 0.03) (layer "F.Cu") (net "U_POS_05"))
 (segment (start 102.828427 101.414214) (end 102.545584 101.697056) (width 0.03) (layer "F.Cu") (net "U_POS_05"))
 (segment (start 101.979899 102.262742) (end 101.697056 102.545584) (width 0.03) (layer "F.Cu") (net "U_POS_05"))
 (segment (start 102.262742 101.979899) (end 101.979899 102.262742) (width 0.03) (layer "F.Cu") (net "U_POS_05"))
 (segment (start 106.788225 97.454416) (end 102.828427 101.414214) (width 0.03) (layer "F.Cu") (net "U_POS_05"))
 (segment (start 101.697056 102.545584) (end 101.414214 102.828427) (width 0.03) (layer "F.Cu") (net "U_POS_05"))
 (segment (start 108.909545 92.646089) (end 106.788225 97.454416) (width 0.03) (layer "F.Cu") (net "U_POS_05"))
 (segment (start 102.545584 101.697056) (end 102.262742 101.979899) (width 0.03) (layer "F.Cu") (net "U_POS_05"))
 (segment (start 100.141421 101.272792) (end 100 101.414214) (width 0.03) (layer "F.Cu") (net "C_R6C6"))
 (segment (start 99.717157 100.848528) (end 100.141421 101.272792) (width 0.03) (layer "F.Cu") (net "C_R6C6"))
 (segment (start 106.929646 90.66619) (end 104.949747 95.615938) (width 0.03) (layer "F.Cu") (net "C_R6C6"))
 (segment (start 107.636753 89.959084) (end 106.929646 90.66619) (width 0.03) (layer "F.Cu") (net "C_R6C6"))
 (segment (start 104.949747 95.615938) (end 99.717157 100.848528) (width 0.03) (layer "F.Cu") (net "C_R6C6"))
 (segment (start 106.081118 89.817662) (end 104.384062 95.050253) (width 0.03) (layer "F.Cu") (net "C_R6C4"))
 (segment (start 99.575736 100.707107) (end 99.434315 100.848528) (width 0.03) (layer "F.Cu") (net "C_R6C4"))
 (segment (start 106.788225 89.110556) (end 106.081118 89.817662) (width 0.03) (layer "F.Cu") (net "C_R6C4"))
 (segment (start 99.151472 100.282843) (end 99.575736 100.707107) (width 0.03) (layer "F.Cu") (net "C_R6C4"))
 (segment (start 104.384062 95.050253) (end 99.151472 100.282843) (width 0.03) (layer "F.Cu") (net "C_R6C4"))
 (segment (start 105.656854 96.323045) (end 101.697056 100.282843) (width 0.03) (layer "F.Cu") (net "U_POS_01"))
 (segment (start 108.485281 90.807612) (end 107.778175 91.514719) (width 0.03) (layer "F.Cu") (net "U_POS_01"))
 (segment (start 100.565685 101.414214) (end 100.282843 101.697056) (width 0.03) (layer "F.Cu") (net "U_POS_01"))
 (segment (start 101.697056 100.282843) (end 101.414214 100.565685) (width 0.03) (layer "F.Cu") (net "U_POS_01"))
 (segment (start 101.131371 100.848528) (end 100.848528 101.131371) (width 0.03) (layer "F.Cu") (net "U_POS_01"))
 (segment (start 101.414214 100.565685) (end 101.131371 100.848528) (width 0.03) (layer "F.Cu") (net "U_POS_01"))
 (segment (start 100.848528 101.131371) (end 100.565685 101.414214) (width 0.03) (layer "F.Cu") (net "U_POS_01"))
 (segment (start 107.778175 91.514719) (end 105.656854 96.323045) (width 0.03) (layer "F.Cu") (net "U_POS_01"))
 (segment (start 110.606602 94.343146) (end 108.485281 99.151472) (width 0.03) (layer "F.Cu") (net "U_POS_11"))
 (segment (start 103.394113 104.242641) (end 103.11127 104.525483) (width 0.03) (layer "F.Cu") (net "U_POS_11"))
 (segment (start 103.959798 103.676955) (end 103.676955 103.959798) (width 0.03) (layer "F.Cu") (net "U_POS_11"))
 (segment (start 104.242641 103.394113) (end 103.959798 103.676955) (width 0.03) (layer "F.Cu") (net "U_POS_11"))
 (segment (start 103.676955 103.959798) (end 103.394113 104.242641) (width 0.03) (layer "F.Cu") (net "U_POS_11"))
 (segment (start 111.313708 93.636039) (end 110.606602 94.343146) (width 0.03) (layer "F.Cu") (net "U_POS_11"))
 (segment (start 104.525483 103.11127) (end 104.242641 103.394113) (width 0.03) (layer "F.Cu") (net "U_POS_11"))
 (segment (start 108.485281 99.151472) (end 104.525483 103.11127) (width 0.03) (layer "F.Cu") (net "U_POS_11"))
 (segment (start 105.798276 89.53482) (end 104.129504 94.795694) (width 0.03) (layer "F.Cu") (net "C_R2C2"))
 (segment (start 106.505382 88.827713) (end 105.798276 89.53482) (width 0.03) (layer "F.Cu") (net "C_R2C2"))
 (segment (start 104.129504 94.795694) (end 100.028284 98.896913) (width 0.03) (layer "F.Cu") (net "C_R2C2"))
 (segment (start 100.028284 98.896913) (end 100.141421 99.010051) (width 0.03) (layer "F.Cu") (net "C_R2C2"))
 (segment (start 100.141421 99.010051) (end 100 99.151472) (width 0.03) (layer "F.Cu") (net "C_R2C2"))
 (segment (start 103.959798 103.11127) (end 103.676955 103.394113) (width 0.03) (layer "F.Cu") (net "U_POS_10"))
 (segment (start 104.242641 102.828427) (end 103.959798 103.11127) (width 0.03) (layer "F.Cu") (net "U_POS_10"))
 (segment (start 103.394113 103.676955) (end 103.11127 103.959798) (width 0.03) (layer "F.Cu") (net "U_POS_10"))
 (segment (start 108.202439 98.868629) (end 104.242641 102.828427) (width 0.03) (layer "F.Cu") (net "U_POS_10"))
 (segment (start 103.11127 103.959798) (end 102.828427 104.242641) (width 0.03) (layer "F.Cu") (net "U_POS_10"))
 (segment (start 110.323759 94.060303) (end 108.202439 98.868629) (width 0.03) (layer "F.Cu") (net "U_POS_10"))
 (segment (start 111.030866 93.353196) (end 110.323759 94.060303) (width 0.03) (layer "F.Cu") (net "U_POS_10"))
 (segment (start 103.676955 103.394113) (end 103.394113 103.676955) (width 0.03) (layer "F.Cu") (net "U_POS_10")))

